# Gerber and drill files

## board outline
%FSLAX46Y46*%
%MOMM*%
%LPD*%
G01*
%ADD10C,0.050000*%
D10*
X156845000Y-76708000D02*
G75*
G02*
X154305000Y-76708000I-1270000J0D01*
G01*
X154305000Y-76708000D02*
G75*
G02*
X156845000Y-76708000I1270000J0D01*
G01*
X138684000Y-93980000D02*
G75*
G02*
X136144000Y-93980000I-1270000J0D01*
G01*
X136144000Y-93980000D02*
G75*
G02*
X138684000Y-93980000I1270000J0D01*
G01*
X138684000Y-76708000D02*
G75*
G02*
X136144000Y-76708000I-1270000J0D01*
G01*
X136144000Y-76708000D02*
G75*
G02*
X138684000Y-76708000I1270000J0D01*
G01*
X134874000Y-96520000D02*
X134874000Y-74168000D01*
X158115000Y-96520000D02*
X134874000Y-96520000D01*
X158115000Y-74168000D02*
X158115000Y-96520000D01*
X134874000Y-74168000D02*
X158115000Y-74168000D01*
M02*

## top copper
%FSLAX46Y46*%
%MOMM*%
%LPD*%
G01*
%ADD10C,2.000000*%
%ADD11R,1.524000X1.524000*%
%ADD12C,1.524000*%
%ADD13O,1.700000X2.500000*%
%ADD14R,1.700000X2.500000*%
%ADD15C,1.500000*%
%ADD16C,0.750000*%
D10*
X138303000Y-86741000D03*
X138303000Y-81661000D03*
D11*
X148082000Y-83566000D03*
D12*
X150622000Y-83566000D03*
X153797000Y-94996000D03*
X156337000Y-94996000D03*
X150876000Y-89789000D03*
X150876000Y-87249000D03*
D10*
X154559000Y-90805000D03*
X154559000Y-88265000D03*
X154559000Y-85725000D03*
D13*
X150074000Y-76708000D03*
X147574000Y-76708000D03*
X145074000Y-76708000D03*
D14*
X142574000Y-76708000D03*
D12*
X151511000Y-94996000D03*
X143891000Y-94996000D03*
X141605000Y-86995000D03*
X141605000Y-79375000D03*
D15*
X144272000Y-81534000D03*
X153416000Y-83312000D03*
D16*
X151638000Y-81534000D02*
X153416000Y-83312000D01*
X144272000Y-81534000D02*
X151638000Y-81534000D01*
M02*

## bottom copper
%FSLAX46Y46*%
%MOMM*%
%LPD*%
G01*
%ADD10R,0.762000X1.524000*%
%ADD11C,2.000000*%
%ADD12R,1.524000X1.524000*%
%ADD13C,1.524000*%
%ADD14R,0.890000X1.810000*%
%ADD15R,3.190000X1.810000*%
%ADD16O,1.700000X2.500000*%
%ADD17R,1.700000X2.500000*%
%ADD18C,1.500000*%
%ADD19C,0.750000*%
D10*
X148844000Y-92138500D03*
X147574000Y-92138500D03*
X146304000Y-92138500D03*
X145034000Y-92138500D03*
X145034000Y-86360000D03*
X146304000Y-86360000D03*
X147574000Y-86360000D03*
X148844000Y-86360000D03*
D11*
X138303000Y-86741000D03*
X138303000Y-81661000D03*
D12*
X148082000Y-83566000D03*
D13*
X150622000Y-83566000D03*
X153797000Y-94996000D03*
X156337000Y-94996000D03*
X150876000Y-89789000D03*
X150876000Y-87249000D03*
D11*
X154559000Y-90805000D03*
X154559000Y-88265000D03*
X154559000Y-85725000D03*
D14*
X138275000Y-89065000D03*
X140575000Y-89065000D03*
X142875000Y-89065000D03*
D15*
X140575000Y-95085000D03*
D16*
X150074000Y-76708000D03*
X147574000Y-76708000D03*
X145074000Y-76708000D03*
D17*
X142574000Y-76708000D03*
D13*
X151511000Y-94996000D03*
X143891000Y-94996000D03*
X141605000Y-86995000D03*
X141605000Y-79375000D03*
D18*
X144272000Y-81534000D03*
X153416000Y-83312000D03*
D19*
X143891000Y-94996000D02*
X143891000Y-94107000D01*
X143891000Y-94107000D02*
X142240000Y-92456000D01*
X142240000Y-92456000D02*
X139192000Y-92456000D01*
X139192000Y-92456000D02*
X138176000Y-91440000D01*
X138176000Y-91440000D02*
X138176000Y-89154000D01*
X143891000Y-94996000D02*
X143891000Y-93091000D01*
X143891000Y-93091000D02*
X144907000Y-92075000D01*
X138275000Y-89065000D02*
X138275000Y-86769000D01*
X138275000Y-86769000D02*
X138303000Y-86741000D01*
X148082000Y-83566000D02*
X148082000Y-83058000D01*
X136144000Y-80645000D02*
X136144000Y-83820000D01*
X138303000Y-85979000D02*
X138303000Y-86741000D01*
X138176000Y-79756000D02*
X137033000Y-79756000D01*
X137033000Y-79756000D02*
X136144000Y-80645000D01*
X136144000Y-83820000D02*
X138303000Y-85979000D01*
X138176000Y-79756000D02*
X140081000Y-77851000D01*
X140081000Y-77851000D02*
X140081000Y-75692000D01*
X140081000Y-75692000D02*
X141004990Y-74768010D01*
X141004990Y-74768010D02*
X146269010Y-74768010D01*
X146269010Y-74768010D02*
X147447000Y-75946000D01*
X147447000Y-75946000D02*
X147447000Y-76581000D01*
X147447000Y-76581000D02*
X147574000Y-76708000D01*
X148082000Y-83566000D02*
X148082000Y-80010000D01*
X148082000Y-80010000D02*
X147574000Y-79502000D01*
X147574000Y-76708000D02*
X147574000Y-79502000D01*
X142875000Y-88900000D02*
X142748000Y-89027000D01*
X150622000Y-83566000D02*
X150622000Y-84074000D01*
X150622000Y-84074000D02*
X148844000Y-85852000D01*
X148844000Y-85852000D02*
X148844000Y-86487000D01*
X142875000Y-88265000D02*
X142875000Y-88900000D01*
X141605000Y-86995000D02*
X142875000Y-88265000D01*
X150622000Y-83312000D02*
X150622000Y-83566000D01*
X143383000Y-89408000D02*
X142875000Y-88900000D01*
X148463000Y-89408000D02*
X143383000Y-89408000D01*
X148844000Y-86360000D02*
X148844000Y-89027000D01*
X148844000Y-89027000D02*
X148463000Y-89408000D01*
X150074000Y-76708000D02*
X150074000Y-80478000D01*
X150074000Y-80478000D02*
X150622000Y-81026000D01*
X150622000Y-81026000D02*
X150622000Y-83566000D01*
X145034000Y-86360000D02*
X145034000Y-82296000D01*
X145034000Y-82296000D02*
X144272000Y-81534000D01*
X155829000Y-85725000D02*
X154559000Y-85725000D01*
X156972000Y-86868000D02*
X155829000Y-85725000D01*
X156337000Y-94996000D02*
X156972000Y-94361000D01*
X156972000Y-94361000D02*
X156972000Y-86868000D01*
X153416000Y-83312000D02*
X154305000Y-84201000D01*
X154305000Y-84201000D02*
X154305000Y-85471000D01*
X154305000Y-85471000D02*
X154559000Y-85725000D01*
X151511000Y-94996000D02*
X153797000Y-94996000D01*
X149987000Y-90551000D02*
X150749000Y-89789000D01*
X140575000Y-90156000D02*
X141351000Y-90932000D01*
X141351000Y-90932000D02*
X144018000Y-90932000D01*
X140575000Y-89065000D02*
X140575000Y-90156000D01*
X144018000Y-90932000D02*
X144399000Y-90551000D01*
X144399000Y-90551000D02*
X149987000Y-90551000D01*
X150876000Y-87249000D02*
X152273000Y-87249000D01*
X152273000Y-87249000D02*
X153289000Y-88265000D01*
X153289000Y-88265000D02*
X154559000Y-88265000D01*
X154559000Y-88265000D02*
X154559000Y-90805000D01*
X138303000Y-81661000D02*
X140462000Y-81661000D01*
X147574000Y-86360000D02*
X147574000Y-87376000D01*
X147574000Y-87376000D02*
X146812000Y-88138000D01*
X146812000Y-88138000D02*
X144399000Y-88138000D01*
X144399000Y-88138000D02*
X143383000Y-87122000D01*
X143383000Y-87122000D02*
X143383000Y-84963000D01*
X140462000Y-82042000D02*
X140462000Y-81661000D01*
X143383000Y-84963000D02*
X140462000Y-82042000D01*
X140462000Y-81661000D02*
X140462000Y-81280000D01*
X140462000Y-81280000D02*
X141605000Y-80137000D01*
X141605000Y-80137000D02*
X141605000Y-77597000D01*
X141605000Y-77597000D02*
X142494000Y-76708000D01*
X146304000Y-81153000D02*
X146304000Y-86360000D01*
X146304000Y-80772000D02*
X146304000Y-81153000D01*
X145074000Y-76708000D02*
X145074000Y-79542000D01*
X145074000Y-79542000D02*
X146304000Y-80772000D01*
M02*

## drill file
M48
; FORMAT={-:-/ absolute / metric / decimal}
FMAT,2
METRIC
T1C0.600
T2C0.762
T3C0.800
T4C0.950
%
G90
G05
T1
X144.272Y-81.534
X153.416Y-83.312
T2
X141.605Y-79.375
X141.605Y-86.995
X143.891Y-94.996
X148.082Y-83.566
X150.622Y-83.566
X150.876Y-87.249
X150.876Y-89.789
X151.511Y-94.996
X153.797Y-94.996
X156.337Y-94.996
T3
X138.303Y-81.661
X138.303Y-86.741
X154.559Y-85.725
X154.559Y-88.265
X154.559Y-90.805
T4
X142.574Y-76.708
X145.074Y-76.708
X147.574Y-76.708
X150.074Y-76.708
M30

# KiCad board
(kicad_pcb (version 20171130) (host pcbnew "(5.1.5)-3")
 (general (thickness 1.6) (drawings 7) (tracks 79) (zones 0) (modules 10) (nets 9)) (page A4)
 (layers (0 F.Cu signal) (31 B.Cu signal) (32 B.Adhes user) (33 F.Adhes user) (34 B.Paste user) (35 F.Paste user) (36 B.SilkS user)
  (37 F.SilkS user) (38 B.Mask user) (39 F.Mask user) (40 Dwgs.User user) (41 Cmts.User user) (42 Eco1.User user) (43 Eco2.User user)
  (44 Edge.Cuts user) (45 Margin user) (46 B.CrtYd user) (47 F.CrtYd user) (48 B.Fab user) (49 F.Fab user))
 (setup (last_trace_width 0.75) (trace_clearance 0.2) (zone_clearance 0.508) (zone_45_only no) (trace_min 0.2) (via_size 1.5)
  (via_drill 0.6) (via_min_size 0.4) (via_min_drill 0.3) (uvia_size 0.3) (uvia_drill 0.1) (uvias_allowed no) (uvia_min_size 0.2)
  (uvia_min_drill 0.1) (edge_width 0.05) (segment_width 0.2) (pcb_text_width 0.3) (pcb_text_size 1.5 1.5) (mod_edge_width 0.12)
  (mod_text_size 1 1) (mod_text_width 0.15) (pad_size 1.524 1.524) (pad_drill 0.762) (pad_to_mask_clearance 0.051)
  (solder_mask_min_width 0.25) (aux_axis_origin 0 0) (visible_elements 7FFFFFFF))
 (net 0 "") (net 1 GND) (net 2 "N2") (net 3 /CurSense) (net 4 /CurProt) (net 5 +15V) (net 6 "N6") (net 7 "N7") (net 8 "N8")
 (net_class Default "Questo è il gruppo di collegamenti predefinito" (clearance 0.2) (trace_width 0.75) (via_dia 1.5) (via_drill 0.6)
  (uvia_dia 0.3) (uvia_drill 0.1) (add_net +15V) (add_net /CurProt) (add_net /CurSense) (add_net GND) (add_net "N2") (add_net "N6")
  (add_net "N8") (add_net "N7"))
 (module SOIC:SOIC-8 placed (layer B.Cu) (at 145.034 89.281 180)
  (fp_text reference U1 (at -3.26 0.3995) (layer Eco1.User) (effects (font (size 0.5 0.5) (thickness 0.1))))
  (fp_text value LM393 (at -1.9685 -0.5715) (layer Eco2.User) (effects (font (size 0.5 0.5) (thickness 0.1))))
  (pad 1 smd rect (at -3.81 -2.8575 180) (size 0.762 1.524) (layers B.Cu B.Paste B.Mask))
  (pad 2 smd rect (at -2.54 -2.8575 180) (size 0.762 1.524) (layers B.Cu B.Paste B.Mask))
  (pad 3 smd rect (at -1.27 -2.8575 180) (size 0.762 1.524) (layers B.Cu B.Paste B.Mask))
  (pad 4 smd rect (at 0 -2.8575 180) (size 0.762 1.524) (layers B.Cu B.Paste B.Mask) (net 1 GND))
  (pad 5 smd rect (at 0 2.921 180) (size 0.762 1.524) (layers B.Cu B.Paste B.Mask) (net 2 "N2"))
  (pad 6 smd rect (at -1.27 2.921 180) (size 0.762 1.524) (layers B.Cu B.Paste B.Mask) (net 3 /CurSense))
  (pad 7 smd rect (at -2.54 2.921 180) (size 0.762 1.524) (layers B.Cu B.Paste B.Mask) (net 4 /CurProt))
  (pad 8 smd rect (at -3.81 2.921 180) (size 0.762 1.524) (layers B.Cu B.Paste B.Mask) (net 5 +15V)))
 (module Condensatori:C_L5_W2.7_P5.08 (layer F.Cu) (at 138.303 81.661 270)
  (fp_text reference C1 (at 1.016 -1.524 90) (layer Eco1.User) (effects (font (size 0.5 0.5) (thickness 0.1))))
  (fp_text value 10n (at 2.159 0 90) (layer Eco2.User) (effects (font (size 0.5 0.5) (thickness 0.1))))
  (pad 2 thru_hole circle (at 5.08 0 270) (size 2 2) (drill 0.8) (layers *.Cu *.Mask) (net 1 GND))
  (pad 1 thru_hole circle (at 0 0 270) (size 2 2) (drill 0.8) (layers *.Cu *.Mask) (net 4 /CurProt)))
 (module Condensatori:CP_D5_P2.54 (layer F.Cu) (at 149.352 83.566)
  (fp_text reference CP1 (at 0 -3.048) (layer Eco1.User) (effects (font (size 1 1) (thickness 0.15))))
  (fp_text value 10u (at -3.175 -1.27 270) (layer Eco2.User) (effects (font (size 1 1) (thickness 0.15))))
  (pad 1 thru_hole rect (at -1.27 0) (size 1.524 1.524) (drill 0.762) (layers *.Cu *.Mask) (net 1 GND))
  (pad 2 thru_hole circle (at 1.27 0) (size 1.524 1.524) (drill 0.762) (layers *.Cu *.Mask) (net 5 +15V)))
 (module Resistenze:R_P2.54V (layer F.Cu) (at 156.337 94.996 180)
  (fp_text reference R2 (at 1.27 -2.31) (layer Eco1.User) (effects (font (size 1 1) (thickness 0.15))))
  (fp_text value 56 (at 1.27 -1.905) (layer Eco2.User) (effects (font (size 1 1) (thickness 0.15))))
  (pad 2 thru_hole circle (at 2.54 0 180) (size 1.524 1.524) (drill 0.762) (layers *.Cu *.Mask) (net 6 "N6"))
  (pad 1 thru_hole circle (at 0 0 180) (size 1.524 1.524) (drill 0.762) (layers *.Cu *.Mask) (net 2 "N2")))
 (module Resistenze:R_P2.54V (layer F.Cu) (at 150.876 87.249 270)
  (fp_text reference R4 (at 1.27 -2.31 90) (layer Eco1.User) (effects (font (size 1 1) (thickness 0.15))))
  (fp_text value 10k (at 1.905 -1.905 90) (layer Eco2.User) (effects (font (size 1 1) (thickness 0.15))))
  (pad 2 thru_hole circle (at 2.54 0 270) (size 1.524 1.524) (drill 0.762) (layers *.Cu *.Mask) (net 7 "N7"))
  (pad 1 thru_hole circle (at 0 0 270) (size 1.524 1.524) (drill 0.762) (layers *.Cu *.Mask) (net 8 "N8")))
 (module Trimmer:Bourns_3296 (layer F.Cu) (at 154.559 85.725 90)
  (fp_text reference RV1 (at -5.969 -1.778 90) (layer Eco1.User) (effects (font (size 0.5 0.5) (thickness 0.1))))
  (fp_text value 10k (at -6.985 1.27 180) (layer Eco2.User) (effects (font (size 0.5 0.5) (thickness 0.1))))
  (pad 3 thru_hole circle (at -5.08 0 90) (size 2 2) (drill 0.8) (layers *.Cu *.Mask) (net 8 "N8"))
  (pad 2 thru_hole circle (at -2.54 0 90) (size 2 2) (drill 0.8) (layers *.Cu *.Mask) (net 8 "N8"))
  (pad 1 thru_hole circle (at 0 0 90) (size 2 2) (drill 0.8) (layers *.Cu *.Mask) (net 2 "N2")))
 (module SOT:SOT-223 (layer B.Cu) (at 140.575 92.075 270)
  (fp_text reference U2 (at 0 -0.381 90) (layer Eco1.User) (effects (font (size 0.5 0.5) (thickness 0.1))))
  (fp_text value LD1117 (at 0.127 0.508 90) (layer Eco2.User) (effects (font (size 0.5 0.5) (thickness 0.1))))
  (pad 1 smd rect (at -3.01 2.3 270) (size 1.81 0.89) (layers B.Cu B.Paste B.Mask) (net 1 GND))
  (pad 2 smd rect (at -3.01 0 270) (size 1.81 0.89) (layers B.Cu B.Paste B.Mask) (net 7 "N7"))
  (pad 3 smd rect (at -3.01 -2.3 270) (size 1.81 0.89) (layers B.Cu B.Paste B.Mask) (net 5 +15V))
  (pad 4 smd rect (at 3.01 0 270) (size 1.81 3.19) (layers B.Cu B.Paste B.Mask)))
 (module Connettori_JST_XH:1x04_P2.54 (layer F.Cu) (at 142.574 76.708)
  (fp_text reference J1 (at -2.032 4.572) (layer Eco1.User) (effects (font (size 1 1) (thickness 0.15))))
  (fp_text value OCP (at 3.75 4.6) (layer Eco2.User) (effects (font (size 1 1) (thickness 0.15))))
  (pad 4 thru_hole oval (at 7.5 0) (size 1.7 2.5) (drill 0.95) (layers *.Cu *.Mask) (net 5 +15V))
  (pad 3 thru_hole oval (at 5 0) (size 1.7 2.5) (drill 0.95) (layers *.Cu *.Mask) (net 1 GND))
  (pad 2 thru_hole oval (at 2.5 0) (size 1.7 2.5) (drill 0.95) (layers *.Cu *.Mask) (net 3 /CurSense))
  (pad 1 thru_hole rect (at 0 0) (size 1.7 2.5) (drill 0.95) (layers *.Cu *.Mask) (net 4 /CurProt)))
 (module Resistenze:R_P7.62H (layer F.Cu) (at 147.701 94.996 180)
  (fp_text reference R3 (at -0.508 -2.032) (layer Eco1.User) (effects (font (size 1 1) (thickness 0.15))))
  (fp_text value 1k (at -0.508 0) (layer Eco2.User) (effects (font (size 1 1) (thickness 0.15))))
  (pad 1 thru_hole circle (at -3.81 0 180) (size 1.524 1.524) (drill 0.762) (layers *.Cu *.Mask) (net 6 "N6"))
  (pad 2 thru_hole circle (at 3.81 0 180) (size 1.524 1.524) (drill 0.762) (layers *.Cu *.Mask) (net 1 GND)))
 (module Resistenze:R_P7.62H (layer B.Cu) (at 141.605 83.185 90)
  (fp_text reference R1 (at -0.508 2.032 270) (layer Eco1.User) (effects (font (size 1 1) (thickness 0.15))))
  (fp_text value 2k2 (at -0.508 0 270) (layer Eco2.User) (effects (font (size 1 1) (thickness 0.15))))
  (pad 1 thru_hole circle (at -3.81 0 90) (size 1.524 1.524) (drill 0.762) (layers *.Cu *.Mask) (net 5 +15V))
  (pad 2 thru_hole circle (at 3.81 0 90) (size 1.524 1.524) (drill 0.762) (layers *.Cu *.Mask) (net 4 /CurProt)))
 (gr_circle (center 155.575 76.708) (end 156.845 76.708) (layer Edge.Cuts) (width 0.05))
 (gr_circle (center 137.414 93.98) (end 136.144 93.98) (layer Edge.Cuts) (width 0.05))
 (gr_circle (center 137.414 76.708) (end 136.144 76.708) (layer Edge.Cuts) (width 0.05))
 (gr_line (start 134.874 96.52) (end 134.874 74.168) (layer Edge.Cuts) (width 0.05))
 (gr_line (start 158.115 96.52) (end 134.874 96.52) (layer Edge.Cuts) (width 0.05))
 (gr_line (start 158.115 74.168) (end 158.115 96.52) (layer Edge.Cuts) (width 0.05))
 (gr_line (start 134.874 74.168) (end 158.115 74.168) (layer Edge.Cuts) (width 0.05))
 (segment (start 143.891 94.996) (end 143.891 94.107) (width 0.75) (layer B.Cu) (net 1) (status 10))
 (segment (start 143.891 94.107) (end 142.24 92.456) (width 0.75) (layer B.Cu) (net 1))
 (segment (start 142.24 92.456) (end 139.192 92.456) (width 0.75) (layer B.Cu) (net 1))
 (segment (start 139.192 92.456) (end 138.176 91.44) (width 0.75) (layer B.Cu) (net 1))
 (segment (start 138.176 91.44) (end 138.176 89.154) (width 0.75) (layer B.Cu) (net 1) (status 20))
 (segment (start 143.891 94.996) (end 143.891 93.091) (width 0.75) (layer B.Cu) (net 1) (status 10))
 (segment (start 143.891 93.091) (end 144.907 92.075) (width 0.75) (layer B.Cu) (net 1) (status 20))
 (segment (start 138.275 89.065) (end 138.275 86.769) (width 0.75) (layer B.Cu) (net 1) (status 30))
 (segment (start 138.275 86.769) (end 138.303 86.741) (width 0.75) (layer B.Cu) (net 1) (status 30))
 (segment (start 148.082 83.566) (end 148.082 83.058) (width 0.75) (layer B.Cu) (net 1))
 (segment (start 136.144 80.645) (end 136.144 83.82) (width 0.75) (layer B.Cu) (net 1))
 (segment (start 138.303 85.979) (end 138.303 86.741) (width 0.75) (layer B.Cu) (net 1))
 (segment (start 138.176 79.756) (end 137.033 79.756) (width 0.75) (layer B.Cu) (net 1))
 (segment (start 137.033 79.756) (end 136.144 80.645) (width 0.75) (layer B.Cu) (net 1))
 (segment (start 136.144 83.82) (end 138.303 85.979) (width 0.75) (layer B.Cu) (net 1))
 (segment (start 138.176 79.756) (end 140.081 77.851) (width 0.75) (layer B.Cu) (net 1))
 (segment (start 140.081 77.851) (end 140.081 75.692) (width 0.75) (layer B.Cu) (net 1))
 (segment (start 140.081 75.692) (end 141.00499 74.76801) (width 0.75) (layer B.Cu) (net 1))
 (segment (start 141.00499 74.76801) (end 146.26901 74.76801) (width 0.75) (layer B.Cu) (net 1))
 (segment (start 146.26901 74.76801) (end 147.447 75.946) (width 0.75) (layer B.Cu) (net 1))
 (segment (start 147.447 75.946) (end 147.447 76.581) (width 0.75) (layer B.Cu) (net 1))
 (segment (start 147.447 76.581) (end 147.574 76.708) (width 0.75) (layer B.Cu) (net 1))
 (segment (start 148.082 83.566) (end 148.082 80.01) (width 0.75) (layer B.Cu) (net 1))
 (segment (start 148.082 80.01) (end 147.574 79.502) (width 0.75) (layer B.Cu) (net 1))
 (segment (start 147.574 76.708) (end 147.574 79.502) (width 0.75) (layer B.Cu) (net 1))
 (segment (start 142.875 88.9) (end 142.748 89.027) (width 0.75) (layer B.Cu) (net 5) (status 30))
 (segment (start 150.622 83.566) (end 150.622 84.074) (width 0.75) (layer B.Cu) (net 5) (status 30))
 (segment (start 150.622 84.074) (end 148.844 85.852) (width 0.75) (layer B.Cu) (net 5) (status 30))
 (segment (start 148.844 85.852) (end 148.844 86.487) (width 0.75) (layer B.Cu) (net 5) (status 30))
 (segment (start 142.875 88.265) (end 142.875 88.9) (width 0.75) (layer B.Cu) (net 5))
 (segment (start 141.605 86.995) (end 142.875 88.265) (width 0.75) (layer B.Cu) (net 5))
 (segment (start 150.622 83.312) (end 150.622 83.566) (width 0.75) (layer B.Cu) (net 5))
 (segment (start 143.383 89.408) (end 142.875 88.9) (width 0.75) (layer B.Cu) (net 5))
 (segment (start 148.463 89.408) (end 143.383 89.408) (width 0.75) (layer B.Cu) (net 5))
 (segment (start 148.844 86.36) (end 148.844 89.027) (width 0.75) (layer B.Cu) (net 5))
 (segment (start 148.844 89.027) (end 148.463 89.408) (width 0.75) (layer B.Cu) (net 5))
 (segment (start 150.074 76.708) (end 150.074 80.478) (width 0.75) (layer B.Cu) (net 5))
 (segment (start 150.074 80.478) (end 150.622 81.026) (width 0.75) (layer B.Cu) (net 5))
 (segment (start 150.622 81.026) (end 150.622 83.566) (width 0.75) (layer B.Cu) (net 5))
 (via (at 144.272 81.534) (size 1.5) (drill 0.6) (layers F.Cu B.Cu) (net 2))
 (segment (start 145.034 86.36) (end 145.034 82.296) (width 0.75) (layer B.Cu) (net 2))
 (segment (start 145.034 82.296) (end 144.272 81.534) (width 0.75) (layer B.Cu) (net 2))
 (segment (start 155.829 85.725) (end 154.559 85.725) (width 0.75) (layer B.Cu) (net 2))
 (segment (start 156.972 86.868) (end 155.829 85.725) (width 0.75) (layer B.Cu) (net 2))
 (segment (start 156.337 94.996) (end 156.972 94.361) (width 0.75) (layer B.Cu) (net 2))
 (segment (start 156.972 94.361) (end 156.972 86.868) (width 0.75) (layer B.Cu) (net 2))
 (segment (start 151.638 81.534) (end 153.416 83.312) (width 0.75) (layer F.Cu) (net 2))
 (segment (start 153.416 83.312) (end 154.305 84.201) (width 0.75) (layer B.Cu) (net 2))
 (via (at 153.416 83.312) (size 1.5) (drill 0.6) (layers F.Cu B.Cu) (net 2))
 (segment (start 154.305 84.201) (end 154.305 85.471) (width 0.75) (layer B.Cu) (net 2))
 (segment (start 154.305 85.471) (end 154.559 85.725) (width 0.75) (layer B.Cu) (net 2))
 (segment (start 144.272 81.534) (end 151.638 81.534) (width 0.75) (layer F.Cu) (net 2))
 (segment (start 151.511 94.996) (end 153.797 94.996) (width 0.75) (layer B.Cu) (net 6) (status 30))
 (segment (start 149.987 90.551) (end 150.749 89.789) (width 0.75) (layer B.Cu) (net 7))
 (segment (start 140.575 90.156) (end 141.351 90.932) (width 0.75) (layer B.Cu) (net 7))
 (segment (start 141.351 90.932) (end 144.018 90.932) (width 0.75) (layer B.Cu) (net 7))
 (segment (start 140.575 89.065) (end 140.575 90.156) (width 0.75) (layer B.Cu) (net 7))
 (segment (start 144.018 90.932) (end 144.399 90.551) (width 0.75) (layer B.Cu) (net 7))
 (segment (start 144.399 90.551) (end 149.987 90.551) (width 0.75) (layer B.Cu) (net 7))
 (segment (start 150.876 87.249) (end 152.273 87.249) (width 0.75) (layer B.Cu) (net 8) (status 10))
 (segment (start 152.273 87.249) (end 153.289 88.265) (width 0.75) (layer B.Cu) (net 8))
 (segment (start 153.289 88.265) (end 154.559 88.265) (width 0.75) (layer B.Cu) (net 8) (status 20))
 (segment (start 154.559 88.265) (end 154.559 90.805) (width 0.75) (layer B.Cu) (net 8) (status 30))
 (segment (start 138.303 81.661) (end 140.462 81.661) (width 0.75) (layer B.Cu) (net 4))
 (segment (start 147.574 86.36) (end 147.574 87.376) (width 0.75) (layer B.Cu) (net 4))
 (segment (start 147.574 87.376) (end 146.812 88.138) (width 0.75) (layer B.Cu) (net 4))
 (segment (start 146.812 88.138) (end 144.399 88.138) (width 0.75) (layer B.Cu) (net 4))
 (segment (start 144.399 88.138) (end 143.383 87.122) (width 0.75) (layer B.Cu) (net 4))
 (segment (start 143.383 87.122) (end 143.383 84.963) (width 0.75) (layer B.Cu) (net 4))
 (segment (start 140.462 82.042) (end 140.462 81.661) (width 0.75) (layer B.Cu) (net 4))
 (segment (start 143.383 84.963) (end 140.462 82.042) (width 0.75) (layer B.Cu) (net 4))
 (segment (start 140.462 81.661) (end 140.462 81.28) (width 0.75) (layer B.Cu) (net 4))
 (segment (start 140.462 81.28) (end 141.605 80.137) (width 0.75) (layer B.Cu) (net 4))
 (segment (start 141.605 80.137) (end 141.605 77.597) (width 0.75) (layer B.Cu) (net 4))
 (segment (start 141.605 77.597) (end 142.494 76.708) (width 0.75) (layer B.Cu) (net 4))
 (segment (start 146.304 81.153) (end 146.304 86.36) (width 0.75) (layer B.Cu) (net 3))
 (segment (start 146.304 80.772) (end 146.304 81.153) (width 0.75) (layer B.Cu) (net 3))
 (segment (start 145.074 76.708) (end 145.074 79.542) (width 0.75) (layer B.Cu) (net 3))
 (segment (start 145.074 79.542) (end 146.304 80.772) (width 0.75) (layer B.Cu) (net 3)))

